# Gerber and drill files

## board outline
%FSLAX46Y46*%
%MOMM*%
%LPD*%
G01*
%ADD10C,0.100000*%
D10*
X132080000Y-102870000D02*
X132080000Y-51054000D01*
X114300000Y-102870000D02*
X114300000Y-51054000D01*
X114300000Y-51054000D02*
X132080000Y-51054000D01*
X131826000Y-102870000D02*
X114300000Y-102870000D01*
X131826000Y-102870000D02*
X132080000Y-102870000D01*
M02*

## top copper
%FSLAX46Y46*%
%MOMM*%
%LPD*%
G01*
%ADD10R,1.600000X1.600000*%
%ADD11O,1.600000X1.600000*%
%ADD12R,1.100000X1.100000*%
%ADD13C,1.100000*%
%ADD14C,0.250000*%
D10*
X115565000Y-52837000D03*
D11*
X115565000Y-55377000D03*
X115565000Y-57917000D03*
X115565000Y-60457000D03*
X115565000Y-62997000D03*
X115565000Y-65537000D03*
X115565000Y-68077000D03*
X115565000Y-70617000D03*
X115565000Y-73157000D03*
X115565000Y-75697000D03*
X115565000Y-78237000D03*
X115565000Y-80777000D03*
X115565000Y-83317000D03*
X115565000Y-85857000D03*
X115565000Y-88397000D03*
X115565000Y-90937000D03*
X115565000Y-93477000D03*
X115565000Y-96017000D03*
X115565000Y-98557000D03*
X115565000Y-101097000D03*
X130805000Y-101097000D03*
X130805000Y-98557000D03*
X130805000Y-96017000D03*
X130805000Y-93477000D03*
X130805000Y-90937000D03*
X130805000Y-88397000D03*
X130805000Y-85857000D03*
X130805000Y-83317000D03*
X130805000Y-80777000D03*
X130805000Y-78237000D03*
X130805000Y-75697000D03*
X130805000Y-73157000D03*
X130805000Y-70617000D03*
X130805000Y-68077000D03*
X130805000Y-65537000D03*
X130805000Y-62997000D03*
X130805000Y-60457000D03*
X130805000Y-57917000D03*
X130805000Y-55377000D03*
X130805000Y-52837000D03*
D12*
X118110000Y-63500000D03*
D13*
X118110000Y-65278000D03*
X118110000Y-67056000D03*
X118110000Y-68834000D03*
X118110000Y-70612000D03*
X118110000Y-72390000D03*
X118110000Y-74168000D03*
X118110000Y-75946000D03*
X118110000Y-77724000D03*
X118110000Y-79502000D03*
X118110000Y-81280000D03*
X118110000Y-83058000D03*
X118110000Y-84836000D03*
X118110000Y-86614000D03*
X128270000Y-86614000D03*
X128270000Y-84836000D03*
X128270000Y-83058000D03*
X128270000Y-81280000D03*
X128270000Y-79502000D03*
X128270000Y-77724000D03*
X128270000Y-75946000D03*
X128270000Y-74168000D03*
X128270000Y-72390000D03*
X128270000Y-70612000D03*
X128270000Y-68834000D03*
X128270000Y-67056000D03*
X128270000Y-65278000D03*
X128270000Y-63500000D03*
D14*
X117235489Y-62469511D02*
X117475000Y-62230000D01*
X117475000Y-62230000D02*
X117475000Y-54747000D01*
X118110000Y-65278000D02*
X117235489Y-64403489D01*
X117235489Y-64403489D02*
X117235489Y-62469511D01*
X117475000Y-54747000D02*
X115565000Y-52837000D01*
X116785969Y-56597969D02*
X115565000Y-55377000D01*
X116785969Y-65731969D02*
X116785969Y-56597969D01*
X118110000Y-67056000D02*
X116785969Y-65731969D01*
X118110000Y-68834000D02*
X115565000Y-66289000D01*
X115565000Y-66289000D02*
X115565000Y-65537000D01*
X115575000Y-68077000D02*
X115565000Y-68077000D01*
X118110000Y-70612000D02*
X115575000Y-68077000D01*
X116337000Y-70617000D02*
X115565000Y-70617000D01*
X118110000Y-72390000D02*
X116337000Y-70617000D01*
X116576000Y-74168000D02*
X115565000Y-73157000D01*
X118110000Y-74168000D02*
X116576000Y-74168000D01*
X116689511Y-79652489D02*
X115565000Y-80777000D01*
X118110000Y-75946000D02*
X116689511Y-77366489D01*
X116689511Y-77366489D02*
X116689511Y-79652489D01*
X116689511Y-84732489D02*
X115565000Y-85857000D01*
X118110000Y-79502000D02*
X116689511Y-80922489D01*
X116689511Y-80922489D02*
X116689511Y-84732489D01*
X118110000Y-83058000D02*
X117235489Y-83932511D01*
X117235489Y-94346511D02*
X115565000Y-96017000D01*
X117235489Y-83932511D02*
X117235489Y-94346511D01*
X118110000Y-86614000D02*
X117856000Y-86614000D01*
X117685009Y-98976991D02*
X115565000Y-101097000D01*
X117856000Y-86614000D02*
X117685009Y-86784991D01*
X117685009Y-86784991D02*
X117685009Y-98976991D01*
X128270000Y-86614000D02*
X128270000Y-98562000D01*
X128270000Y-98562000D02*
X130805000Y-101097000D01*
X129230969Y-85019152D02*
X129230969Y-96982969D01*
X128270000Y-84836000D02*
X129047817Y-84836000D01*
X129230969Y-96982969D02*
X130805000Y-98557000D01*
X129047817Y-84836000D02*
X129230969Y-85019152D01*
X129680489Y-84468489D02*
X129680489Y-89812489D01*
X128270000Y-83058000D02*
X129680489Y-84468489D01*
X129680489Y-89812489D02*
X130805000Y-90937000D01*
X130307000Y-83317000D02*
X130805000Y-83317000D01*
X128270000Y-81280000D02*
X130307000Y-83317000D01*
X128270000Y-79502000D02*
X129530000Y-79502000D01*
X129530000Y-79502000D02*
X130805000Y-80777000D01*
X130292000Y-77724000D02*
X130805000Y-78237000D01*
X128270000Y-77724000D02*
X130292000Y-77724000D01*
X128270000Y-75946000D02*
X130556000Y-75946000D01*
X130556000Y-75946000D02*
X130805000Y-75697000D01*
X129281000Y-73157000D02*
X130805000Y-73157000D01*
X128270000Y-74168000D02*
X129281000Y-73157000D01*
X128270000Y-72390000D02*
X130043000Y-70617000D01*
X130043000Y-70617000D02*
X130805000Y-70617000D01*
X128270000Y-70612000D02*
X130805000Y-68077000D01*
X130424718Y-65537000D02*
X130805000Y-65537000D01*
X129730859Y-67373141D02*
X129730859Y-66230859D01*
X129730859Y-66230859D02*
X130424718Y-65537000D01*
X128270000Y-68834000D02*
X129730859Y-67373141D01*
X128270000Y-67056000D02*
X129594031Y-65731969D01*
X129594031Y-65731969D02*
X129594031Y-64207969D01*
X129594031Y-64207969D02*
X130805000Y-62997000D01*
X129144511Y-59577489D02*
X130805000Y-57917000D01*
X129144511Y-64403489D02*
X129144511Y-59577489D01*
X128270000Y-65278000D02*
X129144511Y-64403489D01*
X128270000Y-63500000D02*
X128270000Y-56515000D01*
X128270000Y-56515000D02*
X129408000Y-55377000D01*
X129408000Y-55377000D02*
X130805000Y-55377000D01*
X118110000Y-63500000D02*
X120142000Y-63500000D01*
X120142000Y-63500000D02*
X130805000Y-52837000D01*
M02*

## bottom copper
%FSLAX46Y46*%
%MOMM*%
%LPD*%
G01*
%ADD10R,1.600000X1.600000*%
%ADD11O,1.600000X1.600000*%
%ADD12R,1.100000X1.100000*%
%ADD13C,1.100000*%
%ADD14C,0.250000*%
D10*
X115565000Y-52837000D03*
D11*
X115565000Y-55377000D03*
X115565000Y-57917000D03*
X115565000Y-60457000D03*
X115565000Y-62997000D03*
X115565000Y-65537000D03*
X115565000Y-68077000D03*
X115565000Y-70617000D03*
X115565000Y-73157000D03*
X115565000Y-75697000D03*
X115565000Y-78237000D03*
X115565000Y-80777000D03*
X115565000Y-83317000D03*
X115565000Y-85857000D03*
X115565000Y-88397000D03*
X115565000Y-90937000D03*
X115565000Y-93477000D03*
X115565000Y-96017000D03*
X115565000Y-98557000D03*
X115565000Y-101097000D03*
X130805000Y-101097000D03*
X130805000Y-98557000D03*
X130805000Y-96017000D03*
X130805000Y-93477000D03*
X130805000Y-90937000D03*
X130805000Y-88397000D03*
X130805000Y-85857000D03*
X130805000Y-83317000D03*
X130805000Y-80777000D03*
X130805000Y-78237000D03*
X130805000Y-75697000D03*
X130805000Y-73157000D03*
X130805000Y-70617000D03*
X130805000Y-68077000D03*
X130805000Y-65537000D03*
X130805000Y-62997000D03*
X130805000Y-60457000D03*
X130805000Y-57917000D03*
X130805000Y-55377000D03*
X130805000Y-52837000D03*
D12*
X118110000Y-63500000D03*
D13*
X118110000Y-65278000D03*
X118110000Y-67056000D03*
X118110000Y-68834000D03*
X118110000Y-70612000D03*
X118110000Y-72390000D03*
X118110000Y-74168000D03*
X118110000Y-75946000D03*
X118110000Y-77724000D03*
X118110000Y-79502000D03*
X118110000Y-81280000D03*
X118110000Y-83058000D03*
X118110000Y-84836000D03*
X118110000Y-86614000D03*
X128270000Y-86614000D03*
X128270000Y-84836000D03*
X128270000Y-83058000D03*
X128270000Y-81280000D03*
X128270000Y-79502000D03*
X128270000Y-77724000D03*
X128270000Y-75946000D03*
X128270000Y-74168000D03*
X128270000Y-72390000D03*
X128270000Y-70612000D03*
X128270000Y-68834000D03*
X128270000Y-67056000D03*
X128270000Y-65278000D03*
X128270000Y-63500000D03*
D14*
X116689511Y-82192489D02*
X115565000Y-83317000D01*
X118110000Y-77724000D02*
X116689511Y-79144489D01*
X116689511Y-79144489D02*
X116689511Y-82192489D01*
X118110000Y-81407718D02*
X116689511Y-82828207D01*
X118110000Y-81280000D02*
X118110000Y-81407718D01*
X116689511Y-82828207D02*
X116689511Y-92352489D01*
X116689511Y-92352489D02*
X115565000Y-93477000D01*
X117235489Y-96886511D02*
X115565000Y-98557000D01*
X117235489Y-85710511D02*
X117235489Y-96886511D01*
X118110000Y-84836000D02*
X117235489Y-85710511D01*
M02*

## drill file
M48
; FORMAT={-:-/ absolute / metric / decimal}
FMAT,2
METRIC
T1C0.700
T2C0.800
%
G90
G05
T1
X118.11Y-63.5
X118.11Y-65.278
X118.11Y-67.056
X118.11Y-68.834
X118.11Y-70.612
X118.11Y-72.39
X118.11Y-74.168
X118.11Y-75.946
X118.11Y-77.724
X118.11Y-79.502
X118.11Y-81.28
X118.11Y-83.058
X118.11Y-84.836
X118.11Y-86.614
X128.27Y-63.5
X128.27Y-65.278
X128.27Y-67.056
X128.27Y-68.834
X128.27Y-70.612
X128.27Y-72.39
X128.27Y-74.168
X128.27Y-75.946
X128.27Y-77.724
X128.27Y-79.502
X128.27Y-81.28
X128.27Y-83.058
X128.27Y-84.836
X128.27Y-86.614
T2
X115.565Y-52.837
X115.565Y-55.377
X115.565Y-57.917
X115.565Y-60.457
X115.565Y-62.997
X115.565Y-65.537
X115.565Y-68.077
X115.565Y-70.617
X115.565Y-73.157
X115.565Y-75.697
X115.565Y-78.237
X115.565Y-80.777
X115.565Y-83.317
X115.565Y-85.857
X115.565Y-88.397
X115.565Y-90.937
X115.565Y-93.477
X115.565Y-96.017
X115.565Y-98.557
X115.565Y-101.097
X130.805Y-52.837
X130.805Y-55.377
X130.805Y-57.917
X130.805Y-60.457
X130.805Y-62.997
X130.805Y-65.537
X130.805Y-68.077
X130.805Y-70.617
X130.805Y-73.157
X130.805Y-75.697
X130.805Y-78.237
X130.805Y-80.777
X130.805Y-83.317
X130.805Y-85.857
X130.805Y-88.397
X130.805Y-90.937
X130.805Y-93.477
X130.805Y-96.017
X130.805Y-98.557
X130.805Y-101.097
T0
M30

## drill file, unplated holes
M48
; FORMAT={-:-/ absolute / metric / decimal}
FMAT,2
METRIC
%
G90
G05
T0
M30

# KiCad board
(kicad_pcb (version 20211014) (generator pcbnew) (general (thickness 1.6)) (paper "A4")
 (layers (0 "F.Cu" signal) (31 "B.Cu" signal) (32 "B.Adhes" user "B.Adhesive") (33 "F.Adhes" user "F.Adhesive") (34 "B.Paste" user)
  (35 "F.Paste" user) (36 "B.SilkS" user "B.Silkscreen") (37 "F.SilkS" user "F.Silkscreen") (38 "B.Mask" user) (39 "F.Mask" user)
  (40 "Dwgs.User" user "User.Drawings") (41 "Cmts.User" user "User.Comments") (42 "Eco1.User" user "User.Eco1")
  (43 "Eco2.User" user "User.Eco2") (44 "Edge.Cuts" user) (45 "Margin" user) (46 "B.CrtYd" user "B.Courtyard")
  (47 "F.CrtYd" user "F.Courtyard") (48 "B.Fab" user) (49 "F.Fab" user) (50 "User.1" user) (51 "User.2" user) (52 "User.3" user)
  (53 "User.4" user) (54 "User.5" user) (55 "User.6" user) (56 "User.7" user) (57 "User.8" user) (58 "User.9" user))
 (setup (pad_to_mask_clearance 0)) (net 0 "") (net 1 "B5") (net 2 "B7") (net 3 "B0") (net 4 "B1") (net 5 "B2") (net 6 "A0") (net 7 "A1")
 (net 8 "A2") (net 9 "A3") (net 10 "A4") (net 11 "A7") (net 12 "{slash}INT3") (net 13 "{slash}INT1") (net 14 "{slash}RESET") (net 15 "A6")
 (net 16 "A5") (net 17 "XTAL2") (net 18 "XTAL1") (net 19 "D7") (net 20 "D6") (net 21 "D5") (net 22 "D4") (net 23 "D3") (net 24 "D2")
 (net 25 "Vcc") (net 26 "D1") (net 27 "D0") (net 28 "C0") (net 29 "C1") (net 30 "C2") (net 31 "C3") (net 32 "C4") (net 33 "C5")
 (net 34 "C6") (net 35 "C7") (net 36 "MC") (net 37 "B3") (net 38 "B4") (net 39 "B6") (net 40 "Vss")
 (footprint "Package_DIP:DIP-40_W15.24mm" (layer "F.Cu") (at 115.565 52.837)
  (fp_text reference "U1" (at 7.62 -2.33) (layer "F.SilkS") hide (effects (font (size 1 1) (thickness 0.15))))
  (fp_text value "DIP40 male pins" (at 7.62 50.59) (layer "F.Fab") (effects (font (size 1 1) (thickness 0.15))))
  (pad "1" thru_hole rect locked (at 0 0) (size 1.6 1.6) (drill 0.8) (layers *.Cu *.Mask) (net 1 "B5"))
  (pad "2" thru_hole oval locked (at 0 2.54) (size 1.6 1.6) (drill 0.8) (layers *.Cu *.Mask) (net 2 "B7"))
  (pad "3" thru_hole oval locked (at 0 5.08) (size 1.6 1.6) (drill 0.8) (layers *.Cu *.Mask) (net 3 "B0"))
  (pad "4" thru_hole oval locked (at 0 7.62) (size 1.6 1.6) (drill 0.8) (layers *.Cu *.Mask) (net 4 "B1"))
  (pad "5" thru_hole oval locked (at 0 10.16) (size 1.6 1.6) (drill 0.8) (layers *.Cu *.Mask) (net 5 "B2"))
  (pad "6" thru_hole oval locked (at 0 12.7) (size 1.6 1.6) (drill 0.8) (layers *.Cu *.Mask) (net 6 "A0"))
  (pad "7" thru_hole oval locked (at 0 15.24) (size 1.6 1.6) (drill 0.8) (layers *.Cu *.Mask) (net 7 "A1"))
  (pad "8" thru_hole oval locked (at 0 17.78) (size 1.6 1.6) (drill 0.8) (layers *.Cu *.Mask) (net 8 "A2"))
  (pad "9" thru_hole oval locked (at 0 20.32) (size 1.6 1.6) (drill 0.8) (layers *.Cu *.Mask) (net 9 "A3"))
  (pad "10" thru_hole oval locked (at 0 22.86) (size 1.6 1.6) (drill 0.8) (layers *.Cu *.Mask) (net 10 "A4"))
  (pad "11" thru_hole oval locked (at 0 25.4) (size 1.6 1.6) (drill 0.8) (layers *.Cu *.Mask) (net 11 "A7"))
  (pad "12" thru_hole oval locked (at 0 27.94) (size 1.6 1.6) (drill 0.8) (layers *.Cu *.Mask) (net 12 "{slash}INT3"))
  (pad "13" thru_hole oval locked (at 0 30.48) (size 1.6 1.6) (drill 0.8) (layers *.Cu *.Mask) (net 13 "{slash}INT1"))
  (pad "14" thru_hole oval locked (at 0 33.02) (size 1.6 1.6) (drill 0.8) (layers *.Cu *.Mask) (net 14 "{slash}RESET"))
  (pad "15" thru_hole oval locked (at 0 35.56) (size 1.6 1.6) (drill 0.8) (layers *.Cu *.Mask) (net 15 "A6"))
  (pad "16" thru_hole oval locked (at 0 38.1) (size 1.6 1.6) (drill 0.8) (layers *.Cu *.Mask) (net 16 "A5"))
  (pad "17" thru_hole oval locked (at 0 40.64) (size 1.6 1.6) (drill 0.8) (layers *.Cu *.Mask) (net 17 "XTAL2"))
  (pad "18" thru_hole oval locked (at 0 43.18) (size 1.6 1.6) (drill 0.8) (layers *.Cu *.Mask) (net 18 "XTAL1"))
  (pad "19" thru_hole oval locked (at 0 45.72) (size 1.6 1.6) (drill 0.8) (layers *.Cu *.Mask) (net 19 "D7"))
  (pad "20" thru_hole oval locked (at 0 48.26) (size 1.6 1.6) (drill 0.8) (layers *.Cu *.Mask) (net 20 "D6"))
  (pad "21" thru_hole oval locked (at 15.24 48.26) (size 1.6 1.6) (drill 0.8) (layers *.Cu *.Mask) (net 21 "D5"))
  (pad "22" thru_hole oval locked (at 15.24 45.72) (size 1.6 1.6) (drill 0.8) (layers *.Cu *.Mask) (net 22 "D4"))
  (pad "23" thru_hole oval locked (at 15.24 43.18) (size 1.6 1.6) (drill 0.8) (layers *.Cu *.Mask) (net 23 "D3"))
  (pad "24" thru_hole oval locked (at 15.24 40.64) (size 1.6 1.6) (drill 0.8) (layers *.Cu *.Mask) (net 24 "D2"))
  (pad "25" thru_hole oval locked (at 15.24 38.1) (size 1.6 1.6) (drill 0.8) (layers *.Cu *.Mask) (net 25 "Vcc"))
  (pad "26" thru_hole oval locked (at 15.24 35.56) (size 1.6 1.6) (drill 0.8) (layers *.Cu *.Mask) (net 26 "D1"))
  (pad "27" thru_hole oval locked (at 15.24 33.02) (size 1.6 1.6) (drill 0.8) (layers *.Cu *.Mask) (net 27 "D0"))
  (pad "28" thru_hole oval locked (at 15.24 30.48) (size 1.6 1.6) (drill 0.8) (layers *.Cu *.Mask) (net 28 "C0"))
  (pad "29" thru_hole oval locked (at 15.24 27.94) (size 1.6 1.6) (drill 0.8) (layers *.Cu *.Mask) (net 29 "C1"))
  (pad "30" thru_hole oval locked (at 15.24 25.4) (size 1.6 1.6) (drill 0.8) (layers *.Cu *.Mask) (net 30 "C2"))
  (pad "31" thru_hole oval locked (at 15.24 22.86) (size 1.6 1.6) (drill 0.8) (layers *.Cu *.Mask) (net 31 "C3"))
  (pad "32" thru_hole oval locked (at 15.24 20.32) (size 1.6 1.6) (drill 0.8) (layers *.Cu *.Mask) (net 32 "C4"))
  (pad "33" thru_hole oval locked (at 15.24 17.78) (size 1.6 1.6) (drill 0.8) (layers *.Cu *.Mask) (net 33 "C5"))
  (pad "34" thru_hole oval locked (at 15.24 15.24) (size 1.6 1.6) (drill 0.8) (layers *.Cu *.Mask) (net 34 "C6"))
  (pad "35" thru_hole oval locked (at 15.24 12.7) (size 1.6 1.6) (drill 0.8) (layers *.Cu *.Mask) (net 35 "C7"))
  (pad "36" thru_hole oval locked (at 15.24 10.16) (size 1.6 1.6) (drill 0.8) (layers *.Cu *.Mask) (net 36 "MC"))
  (pad "37" thru_hole oval locked (at 15.24 7.62) (size 1.6 1.6) (drill 0.8) (layers *.Cu *.Mask) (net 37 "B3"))
  (pad "38" thru_hole oval locked (at 15.24 5.08) (size 1.6 1.6) (drill 0.8) (layers *.Cu *.Mask) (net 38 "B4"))
  (pad "39" thru_hole oval locked (at 15.24 2.54) (size 1.6 1.6) (drill 0.8) (layers *.Cu *.Mask) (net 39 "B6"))
  (pad "40" thru_hole oval locked (at 15.24 0) (size 1.6 1.6) (drill 0.8) (layers *.Cu *.Mask) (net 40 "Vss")))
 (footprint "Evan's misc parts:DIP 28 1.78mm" (layer "F.Cu") (at 118.11 63.5)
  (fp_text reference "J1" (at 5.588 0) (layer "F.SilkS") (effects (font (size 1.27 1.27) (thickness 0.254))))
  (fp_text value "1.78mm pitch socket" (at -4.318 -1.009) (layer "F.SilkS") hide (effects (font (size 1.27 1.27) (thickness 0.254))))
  (pad "1" thru_hole rect (at 0 0) (size 1.1 1.1) (drill 0.7) (layers *.Cu *.Mask) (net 40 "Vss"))
  (pad "2" thru_hole circle (at 0 1.778) (size 1.1 1.1) (drill 0.7) (layers *.Cu *.Mask) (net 1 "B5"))
  (pad "3" thru_hole circle (at 0 3.556) (size 1.1 1.1) (drill 0.7) (layers *.Cu *.Mask) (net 2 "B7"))
  (pad "4" thru_hole circle (at 0 5.334) (size 1.1 1.1) (drill 0.7) (layers *.Cu *.Mask) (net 6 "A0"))
  (pad "5" thru_hole circle (at 0 7.112) (size 1.1 1.1) (drill 0.7) (layers *.Cu *.Mask) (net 7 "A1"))
  (pad "6" thru_hole circle (at 0 8.89) (size 1.1 1.1) (drill 0.7) (layers *.Cu *.Mask) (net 8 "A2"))
  (pad "7" thru_hole circle (at 0 10.668) (size 1.1 1.1) (drill 0.7) (layers *.Cu *.Mask) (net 9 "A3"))
  (pad "8" thru_hole circle (at 0 12.446) (size 1.1 1.1) (drill 0.7) (layers *.Cu *.Mask) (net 12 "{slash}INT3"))
  (pad "9" thru_hole circle (at 0 14.224) (size 1.1 1.1) (drill 0.7) (layers *.Cu *.Mask) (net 13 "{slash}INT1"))
  (pad "10" thru_hole circle (at 0 16.002) (size 1.1 1.1) (drill 0.7) (layers *.Cu *.Mask) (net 14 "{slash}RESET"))
  (pad "11" thru_hole circle (at 0 17.78) (size 1.1 1.1) (drill 0.7) (layers *.Cu *.Mask) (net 17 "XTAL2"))
  (pad "12" thru_hole circle (at 0 19.558) (size 1.1 1.1) (drill 0.7) (layers *.Cu *.Mask) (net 18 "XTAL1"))
  (pad "13" thru_hole circle (at 0 21.336) (size 1.1 1.1) (drill 0.7) (layers *.Cu *.Mask) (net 19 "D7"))
  (pad "14" thru_hole circle (at 0 23.114) (size 1.1 1.1) (drill 0.7) (layers *.Cu *.Mask) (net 20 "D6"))
  (pad "15" thru_hole circle (at 10.16 23.114) (size 1.1 1.1) (drill 0.7) (layers *.Cu *.Mask) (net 21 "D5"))
  (pad "16" thru_hole circle (at 10.16 21.336) (size 1.1 1.1) (drill 0.7) (layers *.Cu *.Mask) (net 22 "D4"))
  (pad "17" thru_hole circle (at 10.16 19.558) (size 1.1 1.1) (drill 0.7) (layers *.Cu *.Mask) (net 25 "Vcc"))
  (pad "18" thru_hole circle (at 10.16 17.78) (size 1.1 1.1) (drill 0.7) (layers *.Cu *.Mask) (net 28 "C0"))
  (pad "19" thru_hole circle (at 10.16 16.002) (size 1.1 1.1) (drill 0.7) (layers *.Cu *.Mask) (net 29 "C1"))
  (pad "20" thru_hole circle (at 10.16 14.224) (size 1.1 1.1) (drill 0.7) (layers *.Cu *.Mask) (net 30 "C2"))
  (pad "21" thru_hole circle (at 10.16 12.446) (size 1.1 1.1) (drill 0.7) (layers *.Cu *.Mask) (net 31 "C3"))
  (pad "22" thru_hole circle (at 10.16 10.668) (size 1.1 1.1) (drill 0.7) (layers *.Cu *.Mask) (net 32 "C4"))
  (pad "23" thru_hole circle (at 10.16 8.89) (size 1.1 1.1) (drill 0.7) (layers *.Cu *.Mask) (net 33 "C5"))
  (pad "24" thru_hole circle (at 10.16 7.112) (size 1.1 1.1) (drill 0.7) (layers *.Cu *.Mask) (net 34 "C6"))
  (pad "25" thru_hole circle (at 10.16 5.334) (size 1.1 1.1) (drill 0.7) (layers *.Cu *.Mask) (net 35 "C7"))
  (pad "26" thru_hole circle (at 10.16 3.556) (size 1.1 1.1) (drill 0.7) (layers *.Cu *.Mask) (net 36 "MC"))
  (pad "27" thru_hole circle (at 10.16 1.778) (size 1.1 1.1) (drill 0.7) (layers *.Cu *.Mask) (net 38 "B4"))
  (pad "28" thru_hole circle (at 10.16 0) (size 1.1 1.1) (drill 0.7) (layers *.Cu *.Mask) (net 39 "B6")))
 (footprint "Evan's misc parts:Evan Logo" (layer "F.Cu") (at 123.444 99.568)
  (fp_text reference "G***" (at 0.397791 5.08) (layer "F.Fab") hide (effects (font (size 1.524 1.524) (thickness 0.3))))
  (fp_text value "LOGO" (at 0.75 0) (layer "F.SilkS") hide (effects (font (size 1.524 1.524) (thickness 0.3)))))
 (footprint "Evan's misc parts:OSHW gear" (layer "B.Cu") (at 123.444 98.552 180)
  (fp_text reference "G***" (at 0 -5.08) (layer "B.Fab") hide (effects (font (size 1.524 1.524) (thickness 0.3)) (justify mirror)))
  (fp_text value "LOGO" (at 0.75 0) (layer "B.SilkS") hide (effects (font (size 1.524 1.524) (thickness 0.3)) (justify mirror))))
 (gr_line (start 132.08 102.87) (end 132.08 51.054) (layer "Edge.Cuts") (width 0.1))
 (gr_line (start 114.3 102.87) (end 114.3 51.054) (layer "Edge.Cuts") (width 0.1))
 (gr_line (start 114.3 51.054) (end 132.08 51.054) (layer "Edge.Cuts") (width 0.1))
 (gr_line (start 131.826 102.87) (end 114.3 102.87) (layer "Edge.Cuts") (width 0.1))
 (gr_line (start 131.826 102.87) (end 132.08 102.87) (layer "Edge.Cuts") (width 0.1))
 (segment (start 117.235489 62.469511) (end 117.475 62.23) (width 0.25) (layer "F.Cu") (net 1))
 (segment (start 117.475 62.23) (end 117.475 54.747) (width 0.25) (layer "F.Cu") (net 1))
 (segment (start 118.11 65.278) (end 117.235489 64.403489) (width 0.25) (layer "F.Cu") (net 1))
 (segment (start 117.235489 64.403489) (end 117.235489 62.469511) (width 0.25) (layer "F.Cu") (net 1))
 (segment (start 117.475 54.747) (end 115.565 52.837) (width 0.25) (layer "F.Cu") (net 1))
 (segment (start 116.785969 56.597969) (end 115.565 55.377) (width 0.25) (layer "F.Cu") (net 2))
 (segment (start 116.785969 65.731969) (end 116.785969 56.597969) (width 0.25) (layer "F.Cu") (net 2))
 (segment (start 118.11 67.056) (end 116.785969 65.731969) (width 0.25) (layer "F.Cu") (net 2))
 (segment (start 118.11 68.834) (end 115.565 66.289) (width 0.25) (layer "F.Cu") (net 6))
 (segment (start 115.565 66.289) (end 115.565 65.537) (width 0.25) (layer "F.Cu") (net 6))
 (segment (start 115.575 68.077) (end 115.565 68.077) (width 0.25) (layer "F.Cu") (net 7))
 (segment (start 118.11 70.612) (end 115.575 68.077) (width 0.25) (layer "F.Cu") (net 7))
 (segment (start 116.337 70.617) (end 115.565 70.617) (width 0.25) (layer "F.Cu") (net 8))
 (segment (start 118.11 72.39) (end 116.337 70.617) (width 0.25) (layer "F.Cu") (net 8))
 (segment (start 116.576 74.168) (end 115.565 73.157) (width 0.25) (layer "F.Cu") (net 9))
 (segment (start 118.11 74.168) (end 116.576 74.168) (width 0.25) (layer "F.Cu") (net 9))
 (segment (start 116.689511 79.652489) (end 115.565 80.777) (width 0.25) (layer "F.Cu") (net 12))
 (segment (start 118.11 75.946) (end 116.689511 77.366489) (width 0.25) (layer "F.Cu") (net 12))
 (segment (start 116.689511 77.366489) (end 116.689511 79.652489) (width 0.25) (layer "F.Cu") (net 12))
 (segment (start 116.689511 82.192489) (end 115.565 83.317) (width 0.25) (layer "B.Cu") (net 13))
 (segment (start 118.11 77.724) (end 116.689511 79.144489) (width 0.25) (layer "B.Cu") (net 13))
 (segment (start 116.689511 79.144489) (end 116.689511 82.192489) (width 0.25) (layer "B.Cu") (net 13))
 (segment (start 116.689511 84.732489) (end 115.565 85.857) (width 0.25) (layer "F.Cu") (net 14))
 (segment (start 118.11 79.502) (end 116.689511 80.922489) (width 0.25) (layer "F.Cu") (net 14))
 (segment (start 116.689511 80.922489) (end 116.689511 84.732489) (width 0.25) (layer "F.Cu") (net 14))
 (segment (start 118.11 81.407718) (end 116.689511 82.828207) (width 0.25) (layer "B.Cu") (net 17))
 (segment (start 118.11 81.28) (end 118.11 81.407718) (width 0.25) (layer "B.Cu") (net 17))
 (segment (start 116.689511 82.828207) (end 116.689511 92.352489) (width 0.25) (layer "B.Cu") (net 17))
 (segment (start 116.689511 92.352489) (end 115.565 93.477) (width 0.25) (layer "B.Cu") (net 17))
 (segment (start 118.11 83.058) (end 117.235489 83.932511) (width 0.25) (layer "F.Cu") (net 18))
 (segment (start 117.235489 94.346511) (end 115.565 96.017) (width 0.25) (layer "F.Cu") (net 18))
 (segment (start 117.235489 83.932511) (end 117.235489 94.346511) (width 0.25) (layer "F.Cu") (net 18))
 (segment (start 117.235489 96.886511) (end 115.565 98.557) (width 0.25) (layer "B.Cu") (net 19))
 (segment (start 117.235489 85.710511) (end 117.235489 96.886511) (width 0.25) (layer "B.Cu") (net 19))
 (segment (start 118.11 84.836) (end 117.235489 85.710511) (width 0.25) (layer "B.Cu") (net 19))
 (segment (start 118.11 86.614) (end 117.856 86.614) (width 0.25) (layer "F.Cu") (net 20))
 (segment (start 117.685009 98.976991) (end 115.565 101.097) (width 0.25) (layer "F.Cu") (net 20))
 (segment (start 117.856 86.614) (end 117.685009 86.784991) (width 0.25) (layer "F.Cu") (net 20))
 (segment (start 117.685009 86.784991) (end 117.685009 98.976991) (width 0.25) (layer "F.Cu") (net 20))
 (segment (start 128.27 86.614) (end 128.27 98.562) (width 0.25) (layer "F.Cu") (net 21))
 (segment (start 128.27 98.562) (end 130.805 101.097) (width 0.25) (layer "F.Cu") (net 21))
 (segment (start 129.230969 85.019152) (end 129.230969 96.982969) (width 0.25) (layer "F.Cu") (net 22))
 (segment (start 128.27 84.836) (end 129.047817 84.836) (width 0.25) (layer "F.Cu") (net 22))
 (segment (start 129.230969 96.982969) (end 130.805 98.557) (width 0.25) (layer "F.Cu") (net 22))
 (segment (start 129.047817 84.836) (end 129.230969 85.019152) (width 0.25) (layer "F.Cu") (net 22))
 (segment (start 129.680489 84.468489) (end 129.680489 89.812489) (width 0.25) (layer "F.Cu") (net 25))
 (segment (start 128.27 83.058) (end 129.680489 84.468489) (width 0.25) (layer "F.Cu") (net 25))
 (segment (start 129.680489 89.812489) (end 130.805 90.937) (width 0.25) (layer "F.Cu") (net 25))
 (segment (start 130.307 83.317) (end 130.805 83.317) (width 0.25) (layer "F.Cu") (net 28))
 (segment (start 128.27 81.28) (end 130.307 83.317) (width 0.25) (layer "F.Cu") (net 28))
 (segment (start 128.27 79.502) (end 129.53 79.502) (width 0.25) (layer "F.Cu") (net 29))
 (segment (start 129.53 79.502) (end 130.805 80.777) (width 0.25) (layer "F.Cu") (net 29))
 (segment (start 130.292 77.724) (end 130.805 78.237) (width 0.25) (layer "F.Cu") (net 30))
 (segment (start 128.27 77.724) (end 130.292 77.724) (width 0.25) (layer "F.Cu") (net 30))
 (segment (start 128.27 75.946) (end 130.556 75.946) (width 0.25) (layer "F.Cu") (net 31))
 (segment (start 130.556 75.946) (end 130.805 75.697) (width 0.25) (layer "F.Cu") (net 31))
 (segment (start 129.281 73.157) (end 130.805 73.157) (width 0.25) (layer "F.Cu") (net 32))
 (segment (start 128.27 74.168) (end 129.281 73.157) (width 0.25) (layer "F.Cu") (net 32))
 (segment (start 128.27 72.39) (end 130.043 70.617) (width 0.25) (layer "F.Cu") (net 33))
 (segment (start 130.043 70.617) (end 130.805 70.617) (width 0.25) (layer "F.Cu") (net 33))
 (segment (start 128.27 70.612) (end 130.805 68.077) (width 0.25) (layer "F.Cu") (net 34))
 (segment (start 130.424718 65.537) (end 130.805 65.537) (width 0.25) (layer "F.Cu") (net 35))
 (segment (start 129.730859 67.373141) (end 129.730859 66.230859) (width 0.25) (layer "F.Cu") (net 35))
 (segment (start 129.730859 66.230859) (end 130.424718 65.537) (width 0.25) (layer "F.Cu") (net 35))
 (segment (start 128.27 68.834) (end 129.730859 67.373141) (width 0.25) (layer "F.Cu") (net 35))
 (segment (start 128.27 67.056) (end 129.594031 65.731969) (width 0.25) (layer "F.Cu") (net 36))
 (segment (start 129.594031 65.731969) (end 129.594031 64.207969) (width 0.25) (layer "F.Cu") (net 36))
 (segment (start 129.594031 64.207969) (end 130.805 62.997) (width 0.25) (layer "F.Cu") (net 36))
 (segment (start 129.144511 59.577489) (end 130.805 57.917) (width 0.25) (layer "F.Cu") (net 38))
 (segment (start 129.144511 64.403489) (end 129.144511 59.577489) (width 0.25) (layer "F.Cu") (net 38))
 (segment (start 128.27 65.278) (end 129.144511 64.403489) (width 0.25) (layer "F.Cu") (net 38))
 (segment (start 128.27 63.5) (end 128.27 56.515) (width 0.25) (layer "F.Cu") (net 39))
 (segment (start 128.27 56.515) (end 129.408 55.377) (width 0.25) (layer "F.Cu") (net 39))
 (segment (start 129.408 55.377) (end 130.805 55.377) (width 0.25) (layer "F.Cu") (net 39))
 (segment (start 118.11 63.5) (end 120.142 63.5) (width 0.25) (layer "F.Cu") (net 40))
 (segment (start 120.142 63.5) (end 130.805 52.837) (width 0.25) (layer "F.Cu") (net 40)))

